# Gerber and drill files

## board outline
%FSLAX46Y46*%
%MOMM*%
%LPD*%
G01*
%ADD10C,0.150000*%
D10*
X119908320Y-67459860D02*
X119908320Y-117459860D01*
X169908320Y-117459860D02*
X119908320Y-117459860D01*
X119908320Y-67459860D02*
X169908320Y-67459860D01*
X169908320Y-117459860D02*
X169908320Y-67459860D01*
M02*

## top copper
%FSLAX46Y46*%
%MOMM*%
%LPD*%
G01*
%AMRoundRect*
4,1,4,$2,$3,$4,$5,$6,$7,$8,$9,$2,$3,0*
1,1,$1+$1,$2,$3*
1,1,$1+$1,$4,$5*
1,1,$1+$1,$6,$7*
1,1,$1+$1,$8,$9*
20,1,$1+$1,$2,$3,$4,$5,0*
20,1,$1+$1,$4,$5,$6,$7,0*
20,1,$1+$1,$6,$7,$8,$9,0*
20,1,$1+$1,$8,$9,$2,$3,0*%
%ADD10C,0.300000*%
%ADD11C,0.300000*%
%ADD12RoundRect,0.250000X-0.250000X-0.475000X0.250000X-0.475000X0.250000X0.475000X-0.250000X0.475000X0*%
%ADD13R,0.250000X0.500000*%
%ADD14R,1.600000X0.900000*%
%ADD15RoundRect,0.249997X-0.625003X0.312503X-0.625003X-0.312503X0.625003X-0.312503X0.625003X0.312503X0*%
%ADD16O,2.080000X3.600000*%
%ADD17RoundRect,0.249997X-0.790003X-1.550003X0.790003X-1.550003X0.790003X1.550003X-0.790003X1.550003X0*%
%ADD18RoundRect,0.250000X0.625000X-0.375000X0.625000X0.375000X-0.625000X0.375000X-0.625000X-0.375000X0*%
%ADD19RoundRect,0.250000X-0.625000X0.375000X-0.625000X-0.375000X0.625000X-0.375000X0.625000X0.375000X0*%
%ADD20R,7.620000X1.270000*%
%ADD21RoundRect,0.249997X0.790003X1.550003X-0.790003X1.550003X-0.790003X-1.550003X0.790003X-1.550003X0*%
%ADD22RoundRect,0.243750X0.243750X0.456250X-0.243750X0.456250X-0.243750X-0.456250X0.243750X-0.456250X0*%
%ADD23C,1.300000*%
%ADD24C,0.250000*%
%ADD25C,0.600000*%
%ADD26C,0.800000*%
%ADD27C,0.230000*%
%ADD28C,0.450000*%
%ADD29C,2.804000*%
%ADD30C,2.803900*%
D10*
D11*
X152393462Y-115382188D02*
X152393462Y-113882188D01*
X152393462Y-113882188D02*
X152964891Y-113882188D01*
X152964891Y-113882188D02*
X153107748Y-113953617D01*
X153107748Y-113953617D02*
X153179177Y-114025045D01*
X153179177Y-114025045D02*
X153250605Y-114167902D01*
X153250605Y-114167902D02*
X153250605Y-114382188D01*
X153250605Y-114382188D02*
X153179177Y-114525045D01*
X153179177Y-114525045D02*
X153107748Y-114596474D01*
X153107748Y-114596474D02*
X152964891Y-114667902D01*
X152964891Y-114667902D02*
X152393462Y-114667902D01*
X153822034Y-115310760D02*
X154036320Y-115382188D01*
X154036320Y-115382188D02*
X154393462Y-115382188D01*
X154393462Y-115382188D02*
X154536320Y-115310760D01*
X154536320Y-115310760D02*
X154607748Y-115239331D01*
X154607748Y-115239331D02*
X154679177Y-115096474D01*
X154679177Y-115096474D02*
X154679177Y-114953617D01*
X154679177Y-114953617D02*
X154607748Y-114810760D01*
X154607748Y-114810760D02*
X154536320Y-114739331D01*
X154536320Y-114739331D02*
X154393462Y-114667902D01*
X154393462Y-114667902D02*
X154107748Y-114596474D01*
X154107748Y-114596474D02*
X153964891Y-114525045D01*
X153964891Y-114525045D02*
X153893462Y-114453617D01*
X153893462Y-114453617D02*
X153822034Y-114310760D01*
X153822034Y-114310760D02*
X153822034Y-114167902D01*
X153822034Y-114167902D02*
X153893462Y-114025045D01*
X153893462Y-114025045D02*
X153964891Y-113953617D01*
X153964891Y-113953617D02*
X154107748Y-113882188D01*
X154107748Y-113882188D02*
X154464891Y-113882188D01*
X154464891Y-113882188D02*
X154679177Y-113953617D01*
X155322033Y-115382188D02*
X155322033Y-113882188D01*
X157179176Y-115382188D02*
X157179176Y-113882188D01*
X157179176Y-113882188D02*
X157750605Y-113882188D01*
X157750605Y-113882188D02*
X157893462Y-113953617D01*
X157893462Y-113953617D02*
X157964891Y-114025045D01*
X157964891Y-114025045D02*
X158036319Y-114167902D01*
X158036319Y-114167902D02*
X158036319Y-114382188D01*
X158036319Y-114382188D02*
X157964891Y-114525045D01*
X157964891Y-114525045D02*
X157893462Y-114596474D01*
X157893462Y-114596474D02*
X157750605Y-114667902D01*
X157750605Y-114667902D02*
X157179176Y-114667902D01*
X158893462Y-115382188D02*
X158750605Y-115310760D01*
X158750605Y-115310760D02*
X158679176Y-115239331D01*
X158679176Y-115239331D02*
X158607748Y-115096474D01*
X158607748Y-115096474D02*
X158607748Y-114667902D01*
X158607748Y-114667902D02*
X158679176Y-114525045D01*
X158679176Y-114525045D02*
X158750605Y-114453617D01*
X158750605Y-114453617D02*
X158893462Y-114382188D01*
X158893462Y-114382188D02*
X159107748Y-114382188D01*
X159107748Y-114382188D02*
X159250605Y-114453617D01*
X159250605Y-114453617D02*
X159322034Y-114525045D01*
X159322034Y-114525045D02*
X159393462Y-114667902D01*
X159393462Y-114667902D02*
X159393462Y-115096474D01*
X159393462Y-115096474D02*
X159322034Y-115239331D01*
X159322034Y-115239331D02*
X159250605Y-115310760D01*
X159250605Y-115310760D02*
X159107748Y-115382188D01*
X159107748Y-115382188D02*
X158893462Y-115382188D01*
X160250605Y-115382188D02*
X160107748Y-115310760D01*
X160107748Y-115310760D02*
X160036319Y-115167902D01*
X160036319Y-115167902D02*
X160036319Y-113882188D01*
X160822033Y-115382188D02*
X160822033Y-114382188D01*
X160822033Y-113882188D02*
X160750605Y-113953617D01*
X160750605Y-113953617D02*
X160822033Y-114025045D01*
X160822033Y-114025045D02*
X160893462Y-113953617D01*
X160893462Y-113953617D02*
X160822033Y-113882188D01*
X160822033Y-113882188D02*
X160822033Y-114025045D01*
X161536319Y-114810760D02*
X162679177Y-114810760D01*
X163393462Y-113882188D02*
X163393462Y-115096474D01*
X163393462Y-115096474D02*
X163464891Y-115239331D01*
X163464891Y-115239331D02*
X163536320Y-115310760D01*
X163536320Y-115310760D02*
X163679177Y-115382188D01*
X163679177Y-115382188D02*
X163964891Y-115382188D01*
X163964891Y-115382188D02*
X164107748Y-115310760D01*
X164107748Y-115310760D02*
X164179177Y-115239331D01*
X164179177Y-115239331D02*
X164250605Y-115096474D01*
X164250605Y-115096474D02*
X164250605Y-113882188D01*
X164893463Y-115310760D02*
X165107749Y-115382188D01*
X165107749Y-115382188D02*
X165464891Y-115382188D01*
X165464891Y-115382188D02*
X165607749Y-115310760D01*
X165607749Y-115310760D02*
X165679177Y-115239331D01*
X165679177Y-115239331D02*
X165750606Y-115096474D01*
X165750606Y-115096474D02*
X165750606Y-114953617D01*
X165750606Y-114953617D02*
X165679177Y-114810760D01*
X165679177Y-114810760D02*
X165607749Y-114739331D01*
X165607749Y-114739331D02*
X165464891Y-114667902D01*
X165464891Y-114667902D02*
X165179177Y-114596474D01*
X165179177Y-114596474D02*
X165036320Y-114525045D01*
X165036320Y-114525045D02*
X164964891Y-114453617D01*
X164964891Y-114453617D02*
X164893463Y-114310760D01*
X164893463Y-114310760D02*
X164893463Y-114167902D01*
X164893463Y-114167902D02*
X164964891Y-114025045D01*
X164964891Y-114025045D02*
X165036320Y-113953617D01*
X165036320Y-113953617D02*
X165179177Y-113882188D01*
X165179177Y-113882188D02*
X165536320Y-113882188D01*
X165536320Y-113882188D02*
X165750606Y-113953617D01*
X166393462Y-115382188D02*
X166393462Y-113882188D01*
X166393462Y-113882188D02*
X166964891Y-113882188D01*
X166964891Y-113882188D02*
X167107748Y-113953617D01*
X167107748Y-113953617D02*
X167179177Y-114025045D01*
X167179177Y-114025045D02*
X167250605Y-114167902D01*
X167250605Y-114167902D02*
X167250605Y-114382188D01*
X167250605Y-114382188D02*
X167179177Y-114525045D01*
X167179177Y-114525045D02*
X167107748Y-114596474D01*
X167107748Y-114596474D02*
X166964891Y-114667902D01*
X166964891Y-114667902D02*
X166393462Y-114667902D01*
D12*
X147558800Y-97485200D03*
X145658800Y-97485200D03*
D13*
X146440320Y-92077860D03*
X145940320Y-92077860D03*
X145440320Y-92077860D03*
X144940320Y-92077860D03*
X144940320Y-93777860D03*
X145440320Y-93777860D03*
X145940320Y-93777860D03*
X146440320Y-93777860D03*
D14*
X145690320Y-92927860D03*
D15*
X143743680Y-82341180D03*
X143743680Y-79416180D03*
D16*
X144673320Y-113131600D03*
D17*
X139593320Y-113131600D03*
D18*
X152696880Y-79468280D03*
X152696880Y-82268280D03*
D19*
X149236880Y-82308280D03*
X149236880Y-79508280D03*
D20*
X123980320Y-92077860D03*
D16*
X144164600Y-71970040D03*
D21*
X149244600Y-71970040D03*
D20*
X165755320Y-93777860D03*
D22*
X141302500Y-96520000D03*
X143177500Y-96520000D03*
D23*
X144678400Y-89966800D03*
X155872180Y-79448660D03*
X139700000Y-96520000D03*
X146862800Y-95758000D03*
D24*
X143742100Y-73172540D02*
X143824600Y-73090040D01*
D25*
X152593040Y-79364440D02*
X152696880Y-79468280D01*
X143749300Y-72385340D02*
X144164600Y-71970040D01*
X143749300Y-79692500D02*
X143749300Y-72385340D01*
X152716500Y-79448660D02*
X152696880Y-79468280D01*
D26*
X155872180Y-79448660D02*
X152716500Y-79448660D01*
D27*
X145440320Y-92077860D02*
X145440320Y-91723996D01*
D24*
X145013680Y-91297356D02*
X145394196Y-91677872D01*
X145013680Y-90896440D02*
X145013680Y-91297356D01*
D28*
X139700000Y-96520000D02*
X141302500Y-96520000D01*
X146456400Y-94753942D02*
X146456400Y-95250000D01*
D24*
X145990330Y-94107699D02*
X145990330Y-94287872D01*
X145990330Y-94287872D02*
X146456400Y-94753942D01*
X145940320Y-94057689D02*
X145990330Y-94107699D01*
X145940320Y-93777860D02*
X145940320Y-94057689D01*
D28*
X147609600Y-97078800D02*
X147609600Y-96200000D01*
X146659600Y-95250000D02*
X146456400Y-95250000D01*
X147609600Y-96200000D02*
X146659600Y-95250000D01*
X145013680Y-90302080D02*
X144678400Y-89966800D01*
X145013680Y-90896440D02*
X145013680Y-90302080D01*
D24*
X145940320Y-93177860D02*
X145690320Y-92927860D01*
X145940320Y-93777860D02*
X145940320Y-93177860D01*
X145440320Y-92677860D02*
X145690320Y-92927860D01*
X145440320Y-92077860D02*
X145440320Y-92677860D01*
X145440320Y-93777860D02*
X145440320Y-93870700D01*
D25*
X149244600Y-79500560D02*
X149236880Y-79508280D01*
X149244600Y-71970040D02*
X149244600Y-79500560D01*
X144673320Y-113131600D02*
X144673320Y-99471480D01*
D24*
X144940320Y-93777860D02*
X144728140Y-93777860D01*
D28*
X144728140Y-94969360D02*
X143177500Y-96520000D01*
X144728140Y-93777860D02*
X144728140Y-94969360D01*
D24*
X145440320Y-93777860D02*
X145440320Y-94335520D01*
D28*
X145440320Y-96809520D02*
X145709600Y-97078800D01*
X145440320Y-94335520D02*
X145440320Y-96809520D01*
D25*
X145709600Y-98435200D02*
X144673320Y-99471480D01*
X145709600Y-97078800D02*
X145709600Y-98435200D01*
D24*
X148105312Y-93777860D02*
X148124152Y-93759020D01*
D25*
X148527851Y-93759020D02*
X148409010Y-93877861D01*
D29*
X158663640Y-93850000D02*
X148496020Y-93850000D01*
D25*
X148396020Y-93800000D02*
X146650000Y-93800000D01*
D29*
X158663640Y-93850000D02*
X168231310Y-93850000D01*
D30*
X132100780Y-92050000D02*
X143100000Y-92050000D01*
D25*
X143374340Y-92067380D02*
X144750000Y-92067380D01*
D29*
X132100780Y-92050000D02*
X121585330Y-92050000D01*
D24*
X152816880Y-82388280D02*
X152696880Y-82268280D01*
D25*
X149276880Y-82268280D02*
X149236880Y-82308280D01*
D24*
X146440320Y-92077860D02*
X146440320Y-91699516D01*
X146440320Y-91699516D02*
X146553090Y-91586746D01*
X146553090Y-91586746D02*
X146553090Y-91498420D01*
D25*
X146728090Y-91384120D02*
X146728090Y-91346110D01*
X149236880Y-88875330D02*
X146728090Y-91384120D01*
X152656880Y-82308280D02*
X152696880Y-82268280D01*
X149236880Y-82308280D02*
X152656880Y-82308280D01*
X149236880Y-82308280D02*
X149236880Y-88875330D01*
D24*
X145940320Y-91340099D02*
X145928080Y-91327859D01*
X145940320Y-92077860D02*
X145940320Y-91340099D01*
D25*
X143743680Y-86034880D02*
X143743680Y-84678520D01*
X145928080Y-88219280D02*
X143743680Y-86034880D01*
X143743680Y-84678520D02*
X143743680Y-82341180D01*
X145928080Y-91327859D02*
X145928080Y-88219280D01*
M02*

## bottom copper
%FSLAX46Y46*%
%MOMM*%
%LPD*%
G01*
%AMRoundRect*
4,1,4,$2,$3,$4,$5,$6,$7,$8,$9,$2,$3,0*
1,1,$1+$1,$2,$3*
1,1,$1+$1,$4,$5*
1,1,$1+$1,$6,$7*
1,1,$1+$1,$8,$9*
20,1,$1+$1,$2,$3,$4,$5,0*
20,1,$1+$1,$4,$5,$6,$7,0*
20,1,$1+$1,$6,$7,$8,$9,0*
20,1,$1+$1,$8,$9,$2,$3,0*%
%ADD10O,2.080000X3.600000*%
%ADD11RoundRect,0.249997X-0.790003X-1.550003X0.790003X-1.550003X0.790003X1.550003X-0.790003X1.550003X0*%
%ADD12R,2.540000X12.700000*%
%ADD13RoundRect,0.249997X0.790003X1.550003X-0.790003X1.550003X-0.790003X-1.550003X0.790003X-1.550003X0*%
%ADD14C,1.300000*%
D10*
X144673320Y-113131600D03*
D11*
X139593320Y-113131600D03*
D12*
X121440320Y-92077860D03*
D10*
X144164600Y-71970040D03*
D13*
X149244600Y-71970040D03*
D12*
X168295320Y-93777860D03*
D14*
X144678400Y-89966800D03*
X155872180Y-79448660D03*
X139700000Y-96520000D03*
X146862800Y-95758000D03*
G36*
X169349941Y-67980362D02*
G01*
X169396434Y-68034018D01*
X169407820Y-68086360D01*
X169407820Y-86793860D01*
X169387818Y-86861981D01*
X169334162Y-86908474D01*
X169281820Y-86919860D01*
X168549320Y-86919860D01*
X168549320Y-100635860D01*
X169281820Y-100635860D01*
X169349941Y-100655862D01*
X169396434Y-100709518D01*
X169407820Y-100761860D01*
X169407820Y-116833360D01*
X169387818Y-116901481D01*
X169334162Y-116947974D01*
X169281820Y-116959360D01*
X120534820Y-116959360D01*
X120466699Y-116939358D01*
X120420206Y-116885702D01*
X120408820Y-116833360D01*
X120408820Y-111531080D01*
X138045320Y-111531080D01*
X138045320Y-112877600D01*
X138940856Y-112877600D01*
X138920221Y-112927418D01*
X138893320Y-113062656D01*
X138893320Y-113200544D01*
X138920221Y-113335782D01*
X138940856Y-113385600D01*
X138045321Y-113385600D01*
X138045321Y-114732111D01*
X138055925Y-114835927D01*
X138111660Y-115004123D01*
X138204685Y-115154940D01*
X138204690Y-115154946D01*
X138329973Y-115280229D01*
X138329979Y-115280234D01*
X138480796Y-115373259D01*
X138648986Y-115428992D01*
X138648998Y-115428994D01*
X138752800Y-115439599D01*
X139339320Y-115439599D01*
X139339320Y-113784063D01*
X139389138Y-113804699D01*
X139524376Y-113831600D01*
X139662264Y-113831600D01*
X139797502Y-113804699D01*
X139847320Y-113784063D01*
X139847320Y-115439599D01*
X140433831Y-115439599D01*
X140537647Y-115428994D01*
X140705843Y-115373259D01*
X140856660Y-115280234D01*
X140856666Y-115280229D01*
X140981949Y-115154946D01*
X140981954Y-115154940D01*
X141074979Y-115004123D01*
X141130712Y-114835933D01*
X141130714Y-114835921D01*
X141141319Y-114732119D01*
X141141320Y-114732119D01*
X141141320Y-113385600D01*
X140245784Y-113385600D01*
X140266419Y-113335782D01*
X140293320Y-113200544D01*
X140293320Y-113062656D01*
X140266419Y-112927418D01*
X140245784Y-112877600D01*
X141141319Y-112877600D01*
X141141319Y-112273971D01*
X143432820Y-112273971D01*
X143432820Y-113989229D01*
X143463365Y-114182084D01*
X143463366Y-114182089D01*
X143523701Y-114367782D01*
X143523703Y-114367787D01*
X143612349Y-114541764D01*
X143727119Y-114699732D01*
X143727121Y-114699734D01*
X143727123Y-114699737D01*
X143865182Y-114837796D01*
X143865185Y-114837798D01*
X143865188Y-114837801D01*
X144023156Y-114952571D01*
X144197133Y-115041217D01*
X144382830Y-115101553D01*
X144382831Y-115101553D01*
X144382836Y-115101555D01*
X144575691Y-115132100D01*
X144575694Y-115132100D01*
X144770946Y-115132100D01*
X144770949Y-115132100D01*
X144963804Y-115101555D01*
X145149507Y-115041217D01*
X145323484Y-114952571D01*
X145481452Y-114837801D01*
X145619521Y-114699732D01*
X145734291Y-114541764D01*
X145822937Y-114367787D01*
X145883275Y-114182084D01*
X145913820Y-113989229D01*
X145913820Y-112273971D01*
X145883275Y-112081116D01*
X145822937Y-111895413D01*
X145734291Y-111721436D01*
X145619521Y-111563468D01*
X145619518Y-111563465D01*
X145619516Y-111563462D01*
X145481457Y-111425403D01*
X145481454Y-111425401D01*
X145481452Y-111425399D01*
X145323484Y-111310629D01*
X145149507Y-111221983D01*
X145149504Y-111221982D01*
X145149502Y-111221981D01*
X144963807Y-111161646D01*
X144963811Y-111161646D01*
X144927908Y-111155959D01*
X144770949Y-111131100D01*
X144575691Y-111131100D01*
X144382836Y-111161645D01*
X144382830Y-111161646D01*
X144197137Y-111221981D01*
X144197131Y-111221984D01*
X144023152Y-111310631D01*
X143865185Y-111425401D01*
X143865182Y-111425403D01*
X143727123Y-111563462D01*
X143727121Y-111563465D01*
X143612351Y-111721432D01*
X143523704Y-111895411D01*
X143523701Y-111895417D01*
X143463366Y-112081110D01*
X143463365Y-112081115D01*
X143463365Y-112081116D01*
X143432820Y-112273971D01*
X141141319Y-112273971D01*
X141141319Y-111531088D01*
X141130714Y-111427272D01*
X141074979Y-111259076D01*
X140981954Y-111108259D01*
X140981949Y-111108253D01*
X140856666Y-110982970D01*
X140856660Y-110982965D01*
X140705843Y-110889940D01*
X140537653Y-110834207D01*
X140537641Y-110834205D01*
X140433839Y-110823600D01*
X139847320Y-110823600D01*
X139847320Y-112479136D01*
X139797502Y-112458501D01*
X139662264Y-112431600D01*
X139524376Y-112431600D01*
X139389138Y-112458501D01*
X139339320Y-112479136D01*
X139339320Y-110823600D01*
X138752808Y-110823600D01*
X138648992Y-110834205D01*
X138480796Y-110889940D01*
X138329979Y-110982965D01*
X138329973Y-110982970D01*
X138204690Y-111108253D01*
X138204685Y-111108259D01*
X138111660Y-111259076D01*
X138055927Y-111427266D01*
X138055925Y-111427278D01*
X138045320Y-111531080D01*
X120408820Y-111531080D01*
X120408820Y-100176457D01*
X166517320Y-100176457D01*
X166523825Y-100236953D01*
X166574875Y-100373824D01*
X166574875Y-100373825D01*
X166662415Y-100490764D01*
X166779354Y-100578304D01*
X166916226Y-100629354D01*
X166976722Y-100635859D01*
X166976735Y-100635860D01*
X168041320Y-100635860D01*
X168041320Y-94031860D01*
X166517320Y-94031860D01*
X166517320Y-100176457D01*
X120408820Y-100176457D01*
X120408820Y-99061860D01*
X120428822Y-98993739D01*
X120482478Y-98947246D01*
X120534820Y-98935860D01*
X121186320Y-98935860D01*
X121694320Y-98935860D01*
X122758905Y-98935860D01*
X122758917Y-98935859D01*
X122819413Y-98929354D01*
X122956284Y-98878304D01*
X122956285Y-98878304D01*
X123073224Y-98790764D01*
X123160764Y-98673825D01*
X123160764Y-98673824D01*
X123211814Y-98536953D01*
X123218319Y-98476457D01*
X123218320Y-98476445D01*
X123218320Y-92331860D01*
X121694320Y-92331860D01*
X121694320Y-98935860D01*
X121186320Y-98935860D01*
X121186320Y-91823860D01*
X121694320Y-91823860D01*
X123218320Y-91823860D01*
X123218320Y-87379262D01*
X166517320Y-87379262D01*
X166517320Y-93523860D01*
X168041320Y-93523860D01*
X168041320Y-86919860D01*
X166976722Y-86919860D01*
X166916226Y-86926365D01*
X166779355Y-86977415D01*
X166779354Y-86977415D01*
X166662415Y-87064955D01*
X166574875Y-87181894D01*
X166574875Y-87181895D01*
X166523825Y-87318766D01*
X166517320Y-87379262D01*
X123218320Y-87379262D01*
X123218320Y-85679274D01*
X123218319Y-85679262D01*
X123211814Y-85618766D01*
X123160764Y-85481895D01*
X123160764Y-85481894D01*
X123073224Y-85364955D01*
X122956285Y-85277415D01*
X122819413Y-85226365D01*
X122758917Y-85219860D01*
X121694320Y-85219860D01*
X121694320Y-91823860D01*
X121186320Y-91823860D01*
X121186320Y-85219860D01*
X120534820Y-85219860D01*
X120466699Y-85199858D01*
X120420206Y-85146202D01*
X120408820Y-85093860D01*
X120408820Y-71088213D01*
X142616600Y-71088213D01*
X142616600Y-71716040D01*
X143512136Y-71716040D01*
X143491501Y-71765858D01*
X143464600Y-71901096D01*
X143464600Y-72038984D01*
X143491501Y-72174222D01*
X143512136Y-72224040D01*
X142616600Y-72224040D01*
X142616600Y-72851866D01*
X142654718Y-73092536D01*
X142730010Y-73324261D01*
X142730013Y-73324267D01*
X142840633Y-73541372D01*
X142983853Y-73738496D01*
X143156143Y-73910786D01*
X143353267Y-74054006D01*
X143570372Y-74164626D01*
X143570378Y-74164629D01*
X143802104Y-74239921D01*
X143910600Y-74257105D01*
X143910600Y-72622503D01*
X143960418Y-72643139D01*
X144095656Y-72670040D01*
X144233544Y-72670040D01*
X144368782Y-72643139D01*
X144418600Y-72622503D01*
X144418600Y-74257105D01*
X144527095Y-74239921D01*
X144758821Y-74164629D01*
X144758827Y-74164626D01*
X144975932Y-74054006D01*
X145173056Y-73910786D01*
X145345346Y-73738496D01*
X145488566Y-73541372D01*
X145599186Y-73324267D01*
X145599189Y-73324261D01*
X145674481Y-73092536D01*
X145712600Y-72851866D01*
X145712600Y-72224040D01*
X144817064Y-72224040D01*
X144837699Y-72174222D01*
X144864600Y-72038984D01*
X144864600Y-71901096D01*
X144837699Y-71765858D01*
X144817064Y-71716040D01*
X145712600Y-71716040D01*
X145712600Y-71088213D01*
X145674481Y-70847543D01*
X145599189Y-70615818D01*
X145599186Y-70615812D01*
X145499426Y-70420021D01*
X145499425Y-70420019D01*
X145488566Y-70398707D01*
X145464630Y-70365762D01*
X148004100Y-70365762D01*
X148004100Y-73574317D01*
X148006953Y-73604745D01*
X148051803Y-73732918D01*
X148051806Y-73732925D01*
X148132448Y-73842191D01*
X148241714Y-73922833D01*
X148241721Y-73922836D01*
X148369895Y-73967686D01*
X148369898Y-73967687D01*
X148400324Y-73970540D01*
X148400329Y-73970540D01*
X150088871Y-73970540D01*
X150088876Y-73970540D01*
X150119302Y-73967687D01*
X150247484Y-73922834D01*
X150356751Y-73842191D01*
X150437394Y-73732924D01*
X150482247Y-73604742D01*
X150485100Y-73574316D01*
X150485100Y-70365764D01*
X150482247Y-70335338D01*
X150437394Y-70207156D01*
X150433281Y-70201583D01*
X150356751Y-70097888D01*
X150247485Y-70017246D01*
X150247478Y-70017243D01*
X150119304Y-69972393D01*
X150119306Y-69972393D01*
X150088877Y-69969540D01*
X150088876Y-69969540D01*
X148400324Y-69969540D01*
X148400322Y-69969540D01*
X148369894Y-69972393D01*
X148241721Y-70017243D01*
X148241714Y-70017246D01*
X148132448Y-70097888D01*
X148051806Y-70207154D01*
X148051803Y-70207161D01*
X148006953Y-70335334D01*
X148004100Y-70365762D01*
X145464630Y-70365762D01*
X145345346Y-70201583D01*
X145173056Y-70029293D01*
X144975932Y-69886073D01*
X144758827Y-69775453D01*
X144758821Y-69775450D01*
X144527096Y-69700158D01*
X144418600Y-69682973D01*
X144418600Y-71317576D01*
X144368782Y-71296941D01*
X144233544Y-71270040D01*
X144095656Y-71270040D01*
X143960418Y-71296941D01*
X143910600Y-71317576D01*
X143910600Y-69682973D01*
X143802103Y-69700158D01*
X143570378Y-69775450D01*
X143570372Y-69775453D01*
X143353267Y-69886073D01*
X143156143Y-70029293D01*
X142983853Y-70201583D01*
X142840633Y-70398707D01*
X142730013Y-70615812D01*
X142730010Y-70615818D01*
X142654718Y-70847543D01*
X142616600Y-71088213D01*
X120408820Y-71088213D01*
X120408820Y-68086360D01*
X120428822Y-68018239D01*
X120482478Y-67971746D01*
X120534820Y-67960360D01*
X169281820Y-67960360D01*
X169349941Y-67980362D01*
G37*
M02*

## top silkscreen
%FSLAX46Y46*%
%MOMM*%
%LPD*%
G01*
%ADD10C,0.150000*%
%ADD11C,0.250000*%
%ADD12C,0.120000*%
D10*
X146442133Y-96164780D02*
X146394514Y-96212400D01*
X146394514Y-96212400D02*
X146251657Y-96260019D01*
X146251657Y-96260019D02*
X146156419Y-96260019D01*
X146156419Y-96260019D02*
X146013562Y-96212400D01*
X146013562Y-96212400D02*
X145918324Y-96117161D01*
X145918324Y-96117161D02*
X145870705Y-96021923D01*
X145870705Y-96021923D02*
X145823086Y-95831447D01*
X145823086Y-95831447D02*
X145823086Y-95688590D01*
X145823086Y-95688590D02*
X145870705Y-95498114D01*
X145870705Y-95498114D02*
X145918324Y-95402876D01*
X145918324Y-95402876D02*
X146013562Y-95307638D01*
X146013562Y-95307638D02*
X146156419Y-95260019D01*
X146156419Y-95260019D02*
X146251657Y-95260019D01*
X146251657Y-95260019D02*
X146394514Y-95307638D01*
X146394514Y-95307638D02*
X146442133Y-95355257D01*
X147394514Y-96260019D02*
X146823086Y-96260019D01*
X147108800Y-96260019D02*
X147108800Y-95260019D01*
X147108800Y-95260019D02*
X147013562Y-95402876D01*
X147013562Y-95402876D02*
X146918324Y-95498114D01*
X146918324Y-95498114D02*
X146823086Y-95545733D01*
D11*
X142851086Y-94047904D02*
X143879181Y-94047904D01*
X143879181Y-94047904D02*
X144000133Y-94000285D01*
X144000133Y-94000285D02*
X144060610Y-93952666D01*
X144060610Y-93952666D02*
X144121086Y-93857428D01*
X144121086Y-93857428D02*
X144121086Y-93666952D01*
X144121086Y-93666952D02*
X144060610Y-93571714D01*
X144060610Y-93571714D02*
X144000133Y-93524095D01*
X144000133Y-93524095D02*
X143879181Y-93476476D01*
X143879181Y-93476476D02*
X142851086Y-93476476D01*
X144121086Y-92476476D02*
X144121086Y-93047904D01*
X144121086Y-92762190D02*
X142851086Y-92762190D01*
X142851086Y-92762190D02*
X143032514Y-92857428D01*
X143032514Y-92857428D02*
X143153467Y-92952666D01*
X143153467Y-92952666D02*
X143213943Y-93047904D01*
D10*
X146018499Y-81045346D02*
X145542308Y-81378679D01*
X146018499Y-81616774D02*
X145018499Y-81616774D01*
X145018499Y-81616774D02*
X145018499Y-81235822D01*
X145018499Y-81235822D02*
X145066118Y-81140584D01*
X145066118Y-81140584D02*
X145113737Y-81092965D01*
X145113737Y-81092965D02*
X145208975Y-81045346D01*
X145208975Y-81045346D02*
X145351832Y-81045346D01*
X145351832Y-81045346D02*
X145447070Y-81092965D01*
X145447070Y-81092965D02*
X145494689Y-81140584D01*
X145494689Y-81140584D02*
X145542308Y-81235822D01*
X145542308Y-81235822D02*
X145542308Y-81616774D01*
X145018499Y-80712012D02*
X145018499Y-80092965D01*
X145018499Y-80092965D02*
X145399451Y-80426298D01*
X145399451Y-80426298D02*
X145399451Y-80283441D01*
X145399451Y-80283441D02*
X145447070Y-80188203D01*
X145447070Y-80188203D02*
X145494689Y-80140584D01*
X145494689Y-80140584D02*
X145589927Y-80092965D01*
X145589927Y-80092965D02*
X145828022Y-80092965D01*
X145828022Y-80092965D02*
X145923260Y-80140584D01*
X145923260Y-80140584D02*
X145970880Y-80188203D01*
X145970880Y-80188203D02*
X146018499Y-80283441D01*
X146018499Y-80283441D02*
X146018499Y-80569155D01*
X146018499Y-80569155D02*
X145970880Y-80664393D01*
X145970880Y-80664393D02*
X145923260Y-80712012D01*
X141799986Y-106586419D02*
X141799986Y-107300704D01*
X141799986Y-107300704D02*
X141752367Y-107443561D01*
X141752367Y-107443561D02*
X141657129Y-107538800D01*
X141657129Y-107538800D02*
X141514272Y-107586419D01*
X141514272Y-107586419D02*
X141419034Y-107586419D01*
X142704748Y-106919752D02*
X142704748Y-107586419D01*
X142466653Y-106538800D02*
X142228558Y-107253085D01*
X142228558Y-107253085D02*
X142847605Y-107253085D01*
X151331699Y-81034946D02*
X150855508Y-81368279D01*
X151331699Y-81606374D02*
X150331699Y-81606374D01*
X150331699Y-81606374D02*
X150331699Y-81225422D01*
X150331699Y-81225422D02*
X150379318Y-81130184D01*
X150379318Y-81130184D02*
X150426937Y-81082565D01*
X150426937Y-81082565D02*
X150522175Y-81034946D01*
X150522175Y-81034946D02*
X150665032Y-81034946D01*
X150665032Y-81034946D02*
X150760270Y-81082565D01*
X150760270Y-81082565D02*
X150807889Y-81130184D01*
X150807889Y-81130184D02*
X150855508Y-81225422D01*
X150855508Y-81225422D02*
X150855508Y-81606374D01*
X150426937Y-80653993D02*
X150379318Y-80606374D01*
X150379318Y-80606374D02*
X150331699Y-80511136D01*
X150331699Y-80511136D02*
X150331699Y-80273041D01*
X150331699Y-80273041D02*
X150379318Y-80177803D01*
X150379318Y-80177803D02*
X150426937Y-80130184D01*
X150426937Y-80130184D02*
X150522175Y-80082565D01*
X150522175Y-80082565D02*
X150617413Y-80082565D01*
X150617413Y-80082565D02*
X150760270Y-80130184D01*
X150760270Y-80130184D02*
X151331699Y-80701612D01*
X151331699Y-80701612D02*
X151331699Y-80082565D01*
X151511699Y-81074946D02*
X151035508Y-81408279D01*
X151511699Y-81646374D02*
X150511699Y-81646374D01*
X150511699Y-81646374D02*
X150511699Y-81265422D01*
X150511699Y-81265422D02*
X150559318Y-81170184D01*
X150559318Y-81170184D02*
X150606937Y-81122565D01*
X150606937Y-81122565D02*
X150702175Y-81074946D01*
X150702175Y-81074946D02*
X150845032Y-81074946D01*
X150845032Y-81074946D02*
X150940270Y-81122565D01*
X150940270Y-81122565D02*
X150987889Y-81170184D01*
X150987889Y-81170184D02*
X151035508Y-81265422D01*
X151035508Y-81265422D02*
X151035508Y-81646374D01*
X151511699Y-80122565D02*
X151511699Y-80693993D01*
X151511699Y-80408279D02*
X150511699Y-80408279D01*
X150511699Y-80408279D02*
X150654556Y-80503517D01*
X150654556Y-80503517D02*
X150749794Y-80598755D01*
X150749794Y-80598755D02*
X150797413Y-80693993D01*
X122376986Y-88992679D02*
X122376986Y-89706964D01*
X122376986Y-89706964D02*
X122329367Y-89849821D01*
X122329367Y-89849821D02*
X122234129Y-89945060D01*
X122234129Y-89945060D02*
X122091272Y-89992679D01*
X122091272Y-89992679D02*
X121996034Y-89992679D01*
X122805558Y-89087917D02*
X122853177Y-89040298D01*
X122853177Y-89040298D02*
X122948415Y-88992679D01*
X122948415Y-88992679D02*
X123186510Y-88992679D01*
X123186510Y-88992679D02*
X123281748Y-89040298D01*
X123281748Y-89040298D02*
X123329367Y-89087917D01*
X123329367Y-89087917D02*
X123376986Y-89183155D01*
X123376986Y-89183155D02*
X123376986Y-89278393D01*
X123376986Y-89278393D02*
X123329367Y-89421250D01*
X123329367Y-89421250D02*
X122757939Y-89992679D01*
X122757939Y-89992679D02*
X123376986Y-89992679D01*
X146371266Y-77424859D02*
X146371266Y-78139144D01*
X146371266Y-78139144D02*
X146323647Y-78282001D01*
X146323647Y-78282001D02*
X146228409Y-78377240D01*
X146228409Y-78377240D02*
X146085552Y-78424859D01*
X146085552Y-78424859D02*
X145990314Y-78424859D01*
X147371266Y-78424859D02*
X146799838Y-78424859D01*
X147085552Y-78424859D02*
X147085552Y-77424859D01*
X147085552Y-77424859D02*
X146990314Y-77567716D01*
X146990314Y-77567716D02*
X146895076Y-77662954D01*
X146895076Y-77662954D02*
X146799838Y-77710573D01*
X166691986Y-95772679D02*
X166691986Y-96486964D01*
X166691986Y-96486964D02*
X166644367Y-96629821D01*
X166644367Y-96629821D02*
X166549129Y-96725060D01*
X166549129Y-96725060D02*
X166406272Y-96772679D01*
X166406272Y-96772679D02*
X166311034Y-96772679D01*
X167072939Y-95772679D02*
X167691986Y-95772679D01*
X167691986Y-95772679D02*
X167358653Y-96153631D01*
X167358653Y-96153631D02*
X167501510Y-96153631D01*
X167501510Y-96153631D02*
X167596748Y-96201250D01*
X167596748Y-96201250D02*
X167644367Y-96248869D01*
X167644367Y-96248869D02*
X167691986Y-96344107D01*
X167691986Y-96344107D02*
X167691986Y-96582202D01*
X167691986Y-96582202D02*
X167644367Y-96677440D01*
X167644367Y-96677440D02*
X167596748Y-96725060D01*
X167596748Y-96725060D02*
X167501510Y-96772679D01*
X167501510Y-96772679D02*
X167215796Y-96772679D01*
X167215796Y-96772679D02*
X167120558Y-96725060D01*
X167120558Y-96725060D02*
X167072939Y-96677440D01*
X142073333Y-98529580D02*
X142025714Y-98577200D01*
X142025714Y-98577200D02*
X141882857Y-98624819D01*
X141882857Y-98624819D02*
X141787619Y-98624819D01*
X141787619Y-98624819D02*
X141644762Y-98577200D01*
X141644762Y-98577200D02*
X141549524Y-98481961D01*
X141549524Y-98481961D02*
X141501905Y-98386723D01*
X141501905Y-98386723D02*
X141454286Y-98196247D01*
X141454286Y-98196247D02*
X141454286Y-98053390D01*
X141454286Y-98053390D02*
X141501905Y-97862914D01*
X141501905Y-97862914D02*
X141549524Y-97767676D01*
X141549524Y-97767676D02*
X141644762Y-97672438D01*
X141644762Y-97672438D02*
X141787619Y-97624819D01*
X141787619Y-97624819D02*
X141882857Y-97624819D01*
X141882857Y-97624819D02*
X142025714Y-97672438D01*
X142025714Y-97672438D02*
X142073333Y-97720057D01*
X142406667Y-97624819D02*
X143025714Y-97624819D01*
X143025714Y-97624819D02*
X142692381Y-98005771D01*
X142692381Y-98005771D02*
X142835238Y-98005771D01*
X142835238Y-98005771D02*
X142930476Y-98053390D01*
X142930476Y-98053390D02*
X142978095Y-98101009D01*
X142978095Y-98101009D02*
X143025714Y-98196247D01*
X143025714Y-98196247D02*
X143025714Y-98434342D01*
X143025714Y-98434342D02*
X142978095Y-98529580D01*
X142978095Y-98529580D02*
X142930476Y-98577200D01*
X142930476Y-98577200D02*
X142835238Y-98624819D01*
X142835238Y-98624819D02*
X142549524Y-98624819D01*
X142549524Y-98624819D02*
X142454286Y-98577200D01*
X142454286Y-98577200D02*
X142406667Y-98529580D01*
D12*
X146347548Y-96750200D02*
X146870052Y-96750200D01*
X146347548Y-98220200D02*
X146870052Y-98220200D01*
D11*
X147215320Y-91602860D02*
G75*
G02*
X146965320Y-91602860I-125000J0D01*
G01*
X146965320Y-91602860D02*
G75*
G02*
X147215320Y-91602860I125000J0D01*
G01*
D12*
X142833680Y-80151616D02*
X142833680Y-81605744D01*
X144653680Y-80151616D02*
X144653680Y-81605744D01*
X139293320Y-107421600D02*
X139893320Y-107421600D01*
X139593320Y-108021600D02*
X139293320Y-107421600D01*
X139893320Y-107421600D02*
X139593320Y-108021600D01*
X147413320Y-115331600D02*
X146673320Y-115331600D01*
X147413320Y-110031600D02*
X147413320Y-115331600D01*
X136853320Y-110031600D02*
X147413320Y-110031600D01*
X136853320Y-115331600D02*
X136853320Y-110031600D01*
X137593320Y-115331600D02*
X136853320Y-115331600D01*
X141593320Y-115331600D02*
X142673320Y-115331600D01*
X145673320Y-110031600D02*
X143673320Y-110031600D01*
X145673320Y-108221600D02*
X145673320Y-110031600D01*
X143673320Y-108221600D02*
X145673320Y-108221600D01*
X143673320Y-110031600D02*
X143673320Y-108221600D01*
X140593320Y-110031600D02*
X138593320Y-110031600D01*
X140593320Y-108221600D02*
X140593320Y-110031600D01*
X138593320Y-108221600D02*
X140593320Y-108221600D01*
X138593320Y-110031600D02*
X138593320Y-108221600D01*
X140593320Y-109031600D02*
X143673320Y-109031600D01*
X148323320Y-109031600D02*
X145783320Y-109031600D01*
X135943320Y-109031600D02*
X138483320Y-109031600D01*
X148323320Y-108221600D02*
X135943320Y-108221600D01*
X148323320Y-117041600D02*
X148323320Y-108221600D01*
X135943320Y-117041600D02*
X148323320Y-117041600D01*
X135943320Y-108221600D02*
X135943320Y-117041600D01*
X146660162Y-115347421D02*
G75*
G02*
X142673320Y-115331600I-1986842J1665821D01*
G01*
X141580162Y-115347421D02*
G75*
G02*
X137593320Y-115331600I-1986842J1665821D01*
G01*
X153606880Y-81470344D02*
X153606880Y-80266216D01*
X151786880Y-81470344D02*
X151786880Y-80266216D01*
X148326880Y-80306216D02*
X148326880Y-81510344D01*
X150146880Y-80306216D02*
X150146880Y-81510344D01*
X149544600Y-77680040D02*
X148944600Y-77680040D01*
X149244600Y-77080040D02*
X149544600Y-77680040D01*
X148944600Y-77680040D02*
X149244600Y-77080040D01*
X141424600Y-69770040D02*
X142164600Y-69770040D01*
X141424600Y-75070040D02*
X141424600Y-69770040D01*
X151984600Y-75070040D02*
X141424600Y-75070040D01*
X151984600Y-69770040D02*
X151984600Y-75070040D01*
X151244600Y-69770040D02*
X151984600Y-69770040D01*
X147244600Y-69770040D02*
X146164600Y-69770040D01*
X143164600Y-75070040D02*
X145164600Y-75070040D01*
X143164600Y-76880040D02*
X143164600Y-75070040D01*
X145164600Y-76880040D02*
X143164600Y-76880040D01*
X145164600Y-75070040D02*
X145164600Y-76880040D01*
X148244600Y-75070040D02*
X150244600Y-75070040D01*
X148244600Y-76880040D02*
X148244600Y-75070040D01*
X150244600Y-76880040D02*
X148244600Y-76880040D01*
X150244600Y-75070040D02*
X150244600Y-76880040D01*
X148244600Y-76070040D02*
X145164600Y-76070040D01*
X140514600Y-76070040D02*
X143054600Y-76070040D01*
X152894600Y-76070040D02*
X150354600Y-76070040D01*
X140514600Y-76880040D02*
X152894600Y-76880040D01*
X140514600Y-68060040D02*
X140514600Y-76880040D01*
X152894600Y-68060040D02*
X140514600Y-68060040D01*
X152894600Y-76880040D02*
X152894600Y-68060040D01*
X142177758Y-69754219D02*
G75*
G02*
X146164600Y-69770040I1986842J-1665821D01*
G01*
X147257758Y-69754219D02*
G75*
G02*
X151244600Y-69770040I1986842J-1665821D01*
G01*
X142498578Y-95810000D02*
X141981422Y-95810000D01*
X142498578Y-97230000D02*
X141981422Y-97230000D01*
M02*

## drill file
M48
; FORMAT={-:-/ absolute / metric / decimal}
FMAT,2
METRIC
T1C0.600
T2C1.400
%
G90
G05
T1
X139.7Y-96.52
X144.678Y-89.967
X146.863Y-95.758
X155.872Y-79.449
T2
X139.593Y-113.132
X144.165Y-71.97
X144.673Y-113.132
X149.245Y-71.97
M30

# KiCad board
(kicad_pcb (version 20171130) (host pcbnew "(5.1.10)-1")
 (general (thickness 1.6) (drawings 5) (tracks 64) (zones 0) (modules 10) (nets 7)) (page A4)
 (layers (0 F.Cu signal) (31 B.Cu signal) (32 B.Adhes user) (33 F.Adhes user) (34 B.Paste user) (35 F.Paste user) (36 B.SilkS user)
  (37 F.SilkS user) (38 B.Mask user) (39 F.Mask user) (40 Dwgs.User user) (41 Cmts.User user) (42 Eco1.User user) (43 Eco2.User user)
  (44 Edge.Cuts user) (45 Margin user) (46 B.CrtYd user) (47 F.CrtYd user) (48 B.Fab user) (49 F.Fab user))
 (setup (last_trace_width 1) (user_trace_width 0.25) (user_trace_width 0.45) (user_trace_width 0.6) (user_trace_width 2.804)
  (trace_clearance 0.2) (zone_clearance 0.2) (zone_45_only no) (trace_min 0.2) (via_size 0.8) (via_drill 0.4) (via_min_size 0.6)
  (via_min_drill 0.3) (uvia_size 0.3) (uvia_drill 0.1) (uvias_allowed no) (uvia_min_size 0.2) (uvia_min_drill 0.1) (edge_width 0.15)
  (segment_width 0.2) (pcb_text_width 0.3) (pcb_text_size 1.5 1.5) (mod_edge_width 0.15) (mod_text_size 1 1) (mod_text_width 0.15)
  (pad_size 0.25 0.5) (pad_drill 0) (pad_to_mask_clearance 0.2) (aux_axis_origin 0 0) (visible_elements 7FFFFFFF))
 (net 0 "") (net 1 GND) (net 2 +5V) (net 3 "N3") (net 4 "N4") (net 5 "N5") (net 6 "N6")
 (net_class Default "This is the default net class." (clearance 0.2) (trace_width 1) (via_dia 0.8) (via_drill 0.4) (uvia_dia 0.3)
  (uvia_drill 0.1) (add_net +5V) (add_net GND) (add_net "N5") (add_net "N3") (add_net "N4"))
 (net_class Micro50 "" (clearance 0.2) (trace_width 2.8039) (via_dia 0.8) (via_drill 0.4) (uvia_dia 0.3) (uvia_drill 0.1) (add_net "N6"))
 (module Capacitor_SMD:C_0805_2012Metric (layer F.Cu) (at 146.6088 97.4852)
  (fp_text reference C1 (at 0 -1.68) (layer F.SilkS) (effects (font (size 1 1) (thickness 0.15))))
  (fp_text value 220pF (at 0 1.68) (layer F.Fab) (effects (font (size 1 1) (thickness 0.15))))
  (fp_line (start -0.261252 -0.735) (end 0.261252 -0.735) (layer F.SilkS) (width 0.12))
  (fp_line (start -0.261252 0.735) (end 0.261252 0.735) (layer F.SilkS) (width 0.12))
  (pad 2 smd roundrect (at 0.95 0) (size 1 1.45) (layers F.Cu F.Paste F.Mask) (roundrect_rratio 0.25) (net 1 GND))
  (pad 1 smd roundrect (at -0.95 0) (size 1 1.45) (layers F.Cu F.Paste F.Mask) (roundrect_rratio 0.25) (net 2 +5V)))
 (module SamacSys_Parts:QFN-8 (layer F.Cu) (at 145.69032 92.92786 270)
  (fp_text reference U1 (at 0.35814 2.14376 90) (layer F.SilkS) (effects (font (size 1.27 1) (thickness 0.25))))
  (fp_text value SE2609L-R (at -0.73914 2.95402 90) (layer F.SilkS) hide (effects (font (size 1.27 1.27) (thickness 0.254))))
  (fp_circle (center -1.325 -1.4) (end -1.325 -1.275) (layer F.SilkS) (width 0.25))
  (pad 1 smd rect (at -0.85 -0.75) (size 0.25 0.5) (layers F.Cu F.Paste F.Mask) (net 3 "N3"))
  (pad 2 smd rect (at -0.85 -0.25) (size 0.25 0.5) (layers F.Cu F.Paste F.Mask) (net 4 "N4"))
  (pad 3 smd rect (at -0.85 0.25) (size 0.25 0.5) (layers F.Cu F.Paste F.Mask) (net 1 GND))
  (pad 4 smd rect (at -0.85 0.75) (size 0.25 0.5) (layers F.Cu F.Paste F.Mask) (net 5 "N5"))
  (pad 5 smd rect (at 0.85 0.75) (size 0.25 0.5) (layers F.Cu F.Paste F.Mask) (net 2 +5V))
  (pad 6 smd rect (at 0.85 0.25) (size 0.25 0.5) (layers F.Cu F.Paste F.Mask) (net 2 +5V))
  (pad 7 smd rect (at 0.85 -0.25) (size 0.25 0.5) (layers F.Cu F.Paste F.Mask) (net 1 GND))
  (pad 8 smd rect (at 0.85 -0.75) (size 0.25 0.5) (layers F.Cu F.Paste F.Mask) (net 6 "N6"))
  (pad 9 smd rect (at 0 0 270) (size 0.9 1.6) (layers F.Cu F.Paste F.Mask) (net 1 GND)))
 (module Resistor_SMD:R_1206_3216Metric (layer F.Cu) (at 143.74368 80.87868 270)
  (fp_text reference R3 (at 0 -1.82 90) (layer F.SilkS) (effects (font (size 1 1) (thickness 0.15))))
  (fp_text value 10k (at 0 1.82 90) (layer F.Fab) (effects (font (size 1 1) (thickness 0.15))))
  (fp_line (start -0.727064 0.91) (end 0.727064 0.91) (layer F.SilkS) (width 0.12))
  (fp_line (start -0.727064 -0.91) (end 0.727064 -0.91) (layer F.SilkS) (width 0.12))
  (pad 2 smd roundrect (at 1.4625 0 270) (size 1.125 1.75) (layers F.Cu F.Paste F.Mask) (roundrect_rratio 0.2222195555555556) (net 4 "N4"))
  (pad 1 smd roundrect (at -1.4625 0 270) (size 1.125 1.75) (layers F.Cu F.Paste F.Mask) (roundrect_rratio 0.2222195555555556) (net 1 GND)))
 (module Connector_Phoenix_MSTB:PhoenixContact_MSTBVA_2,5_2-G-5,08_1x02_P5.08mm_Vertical (layer F.Cu) (at 139.59332 113.1316)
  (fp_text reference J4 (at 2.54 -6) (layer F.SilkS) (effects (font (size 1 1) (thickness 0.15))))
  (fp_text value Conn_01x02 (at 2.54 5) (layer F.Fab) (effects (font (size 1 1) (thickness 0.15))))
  (fp_line (start -0.3 -5.71) (end 0.3 -5.71) (layer F.SilkS) (width 0.12))
  (fp_line (start 0 -5.11) (end -0.3 -5.71) (layer F.SilkS) (width 0.12))
  (fp_line (start 0.3 -5.71) (end 0 -5.11) (layer F.SilkS) (width 0.12))
  (fp_line (start 7.82 2.2) (end 7.08 2.2) (layer F.SilkS) (width 0.12))
  (fp_line (start 7.82 -3.1) (end 7.82 2.2) (layer F.SilkS) (width 0.12))
  (fp_line (start -2.74 -3.1) (end 7.82 -3.1) (layer F.SilkS) (width 0.12))
  (fp_line (start -2.74 2.2) (end -2.74 -3.1) (layer F.SilkS) (width 0.12))
  (fp_line (start -2 2.2) (end -2.74 2.2) (layer F.SilkS) (width 0.12))
  (fp_line (start 2 2.2) (end 3.08 2.2) (layer F.SilkS) (width 0.12))
  (fp_line (start 6.08 -3.1) (end 4.08 -3.1) (layer F.SilkS) (width 0.12))
  (fp_line (start 6.08 -4.91) (end 6.08 -3.1) (layer F.SilkS) (width 0.12))
  (fp_line (start 4.08 -4.91) (end 6.08 -4.91) (layer F.SilkS) (width 0.12))
  (fp_line (start 4.08 -3.1) (end 4.08 -4.91) (layer F.SilkS) (width 0.12))
  (fp_line (start 1 -3.1) (end -1 -3.1) (layer F.SilkS) (width 0.12))
  (fp_line (start 1 -4.91) (end 1 -3.1) (layer F.SilkS) (width 0.12))
  (fp_line (start -1 -4.91) (end 1 -4.91) (layer F.SilkS) (width 0.12))
  (fp_line (start -1 -3.1) (end -1 -4.91) (layer F.SilkS) (width 0.12))
  (fp_line (start 1 -4.1) (end 4.08 -4.1) (layer F.SilkS) (width 0.12))
  (fp_line (start 8.73 -4.1) (end 6.19 -4.1) (layer F.SilkS) (width 0.12))
  (fp_line (start -3.65 -4.1) (end -1.11 -4.1) (layer F.SilkS) (width 0.12))
  (fp_line (start 8.73 -4.91) (end -3.65 -4.91) (layer F.SilkS) (width 0.12))
  (fp_line (start 8.73 3.91) (end 8.73 -4.91) (layer F.SilkS) (width 0.12))
  (fp_line (start -3.65 3.91) (end 8.73 3.91) (layer F.SilkS) (width 0.12))
  (fp_line (start -3.65 -4.91) (end -3.65 3.91) (layer F.SilkS) (width 0.12))
  (fp_arc (start 5.08 0.55) (end 3.08 2.2) (angle -100.5) (layer F.SilkS) (width 0.12))
  (fp_arc (start 0 0.55) (end -2 2.2) (angle -100.5) (layer F.SilkS) (width 0.12))
  (pad 2 thru_hole oval (at 5.08 0) (size 2.08 3.6) (drill 1.4) (layers *.Cu *.Mask) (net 2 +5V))
  (pad 1 thru_hole roundrect (at 0 0) (size 2.08 3.6) (drill 1.4) (layers *.Cu *.Mask) (roundrect_rratio 0.1201908653846154) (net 1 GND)))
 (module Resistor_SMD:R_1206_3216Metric (layer F.Cu) (at 152.69688 80.86828 90)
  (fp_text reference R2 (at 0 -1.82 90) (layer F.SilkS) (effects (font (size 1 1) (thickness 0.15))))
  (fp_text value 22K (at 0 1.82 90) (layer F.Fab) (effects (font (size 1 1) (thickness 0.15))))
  (fp_line (start -0.602064 0.91) (end 0.602064 0.91) (layer F.SilkS) (width 0.12))
  (fp_line (start -0.602064 -0.91) (end 0.602064 -0.91) (layer F.SilkS) (width 0.12))
  (pad 2 smd roundrect (at 1.4 0 90) (size 1.25 1.75) (layers F.Cu F.Paste F.Mask) (roundrect_rratio 0.2) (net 1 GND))
  (pad 1 smd roundrect (at -1.4 0 90) (size 1.25 1.75) (layers F.Cu F.Paste F.Mask) (roundrect_rratio 0.2) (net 3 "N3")))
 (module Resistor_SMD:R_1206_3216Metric (layer F.Cu) (at 149.23688 80.90828 270)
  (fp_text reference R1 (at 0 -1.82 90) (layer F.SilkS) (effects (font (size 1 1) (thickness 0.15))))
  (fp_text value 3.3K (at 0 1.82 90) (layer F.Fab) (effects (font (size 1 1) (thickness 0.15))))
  (fp_line (start -0.602064 0.91) (end 0.602064 0.91) (layer F.SilkS) (width 0.12))
  (fp_line (start -0.602064 -0.91) (end 0.602064 -0.91) (layer F.SilkS) (width 0.12))
  (pad 2 smd roundrect (at 1.4 0 270) (size 1.25 1.75) (layers F.Cu F.Paste F.Mask) (roundrect_rratio 0.2) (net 3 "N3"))
  (pad 1 smd roundrect (at -1.4 0 270) (size 1.25 1.75) (layers F.Cu F.Paste F.Mask) (roundrect_rratio 0.2) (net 2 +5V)))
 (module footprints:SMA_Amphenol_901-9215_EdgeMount (layer F.Cu) (at 125.25032 92.07786 180)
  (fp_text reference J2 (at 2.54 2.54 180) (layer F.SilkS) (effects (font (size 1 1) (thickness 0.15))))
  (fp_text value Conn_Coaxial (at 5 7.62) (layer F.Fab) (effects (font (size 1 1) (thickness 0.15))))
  (pad 1 smd rect (at 1.27 0 270) (size 1.27 7.62) (layers F.Cu F.Paste F.Mask) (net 5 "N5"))
  (pad 2 smd rect (at 3.81 0) (size 2.54 12.7) (layers B.Cu B.Paste B.Mask) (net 1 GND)))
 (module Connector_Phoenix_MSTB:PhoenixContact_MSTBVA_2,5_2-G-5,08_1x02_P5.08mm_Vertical (layer F.Cu) (at 149.2446 71.97004 180)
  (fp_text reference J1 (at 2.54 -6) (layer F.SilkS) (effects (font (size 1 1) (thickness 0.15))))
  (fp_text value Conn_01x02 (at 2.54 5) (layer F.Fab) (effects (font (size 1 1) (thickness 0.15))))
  (fp_line (start -0.3 -5.71) (end 0.3 -5.71) (layer F.SilkS) (width 0.12))
  (fp_line (start 0 -5.11) (end -0.3 -5.71) (layer F.SilkS) (width 0.12))
  (fp_line (start 0.3 -5.71) (end 0 -5.11) (layer F.SilkS) (width 0.12))
  (fp_line (start 7.82 2.2) (end 7.08 2.2) (layer F.SilkS) (width 0.12))
  (fp_line (start 7.82 -3.1) (end 7.82 2.2) (layer F.SilkS) (width 0.12))
  (fp_line (start -2.74 -3.1) (end 7.82 -3.1) (layer F.SilkS) (width 0.12))
  (fp_line (start -2.74 2.2) (end -2.74 -3.1) (layer F.SilkS) (width 0.12))
  (fp_line (start -2 2.2) (end -2.74 2.2) (layer F.SilkS) (width 0.12))
  (fp_line (start 2 2.2) (end 3.08 2.2) (layer F.SilkS) (width 0.12))
  (fp_line (start 6.08 -3.1) (end 4.08 -3.1) (layer F.SilkS) (width 0.12))
  (fp_line (start 6.08 -4.91) (end 6.08 -3.1) (layer F.SilkS) (width 0.12))
  (fp_line (start 4.08 -4.91) (end 6.08 -4.91) (layer F.SilkS) (width 0.12))
  (fp_line (start 4.08 -3.1) (end 4.08 -4.91) (layer F.SilkS) (width 0.12))
  (fp_line (start 1 -3.1) (end -1 -3.1) (layer F.SilkS) (width 0.12))
  (fp_line (start 1 -4.91) (end 1 -3.1) (layer F.SilkS) (width 0.12))
  (fp_line (start -1 -4.91) (end 1 -4.91) (layer F.SilkS) (width 0.12))
  (fp_line (start -1 -3.1) (end -1 -4.91) (layer F.SilkS) (width 0.12))
  (fp_line (start 1 -4.1) (end 4.08 -4.1) (layer F.SilkS) (width 0.12))
  (fp_line (start 8.73 -4.1) (end 6.19 -4.1) (layer F.SilkS) (width 0.12))
  (fp_line (start -3.65 -4.1) (end -1.11 -4.1) (layer F.SilkS) (width 0.12))
  (fp_line (start 8.73 -4.91) (end -3.65 -4.91) (layer F.SilkS) (width 0.12))
  (fp_line (start 8.73 3.91) (end 8.73 -4.91) (layer F.SilkS) (width 0.12))
  (fp_line (start -3.65 3.91) (end 8.73 3.91) (layer F.SilkS) (width 0.12))
  (fp_line (start -3.65 -4.91) (end -3.65 3.91) (layer F.SilkS) (width 0.12))
  (fp_arc (start 5.08 0.55) (end 3.08 2.2) (angle -100.5) (layer F.SilkS) (width 0.12))
  (fp_arc (start 0 0.55) (end -2 2.2) (angle -100.5) (layer F.SilkS) (width 0.12))
  (pad 2 thru_hole oval (at 5.08 0 180) (size 2.08 3.6) (drill 1.4) (layers *.Cu *.Mask) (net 1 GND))
  (pad 1 thru_hole roundrect (at 0 0 180) (size 2.08 3.6) (drill 1.4) (layers *.Cu *.Mask) (roundrect_rratio 0.1201908653846154) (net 2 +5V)))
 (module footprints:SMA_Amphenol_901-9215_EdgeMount (layer F.Cu) (at 164.48532 93.77786)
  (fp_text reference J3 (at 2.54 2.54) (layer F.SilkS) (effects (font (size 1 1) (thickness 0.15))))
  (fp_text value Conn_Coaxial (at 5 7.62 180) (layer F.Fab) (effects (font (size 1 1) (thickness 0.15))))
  (pad 1 smd rect (at 1.27 0 90) (size 1.27 7.62) (layers F.Cu F.Paste F.Mask) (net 6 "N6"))
  (pad 2 smd rect (at 3.81 0 180) (size 2.54 12.7) (layers B.Cu B.Paste B.Mask) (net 1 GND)))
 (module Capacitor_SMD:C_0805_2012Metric (layer F.Cu) (at 142.24 96.52 180)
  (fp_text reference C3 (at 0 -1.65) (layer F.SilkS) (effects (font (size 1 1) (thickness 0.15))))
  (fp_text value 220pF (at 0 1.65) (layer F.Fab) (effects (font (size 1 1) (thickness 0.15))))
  (fp_line (start -0.258578 0.71) (end 0.258578 0.71) (layer F.SilkS) (width 0.12))
  (fp_line (start -0.258578 -0.71) (end 0.258578 -0.71) (layer F.SilkS) (width 0.12))
  (pad 2 smd roundrect (at 0.9375 0 180) (size 0.975 1.4) (layers F.Cu F.Paste F.Mask) (roundrect_rratio 0.25) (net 1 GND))
  (pad 1 smd roundrect (at -0.9375 0 180) (size 0.975 1.4) (layers F.Cu F.Paste F.Mask) (roundrect_rratio 0.25) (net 2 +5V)))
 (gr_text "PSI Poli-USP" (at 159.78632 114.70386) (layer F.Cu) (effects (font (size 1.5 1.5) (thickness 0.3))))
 (gr_line (start 119.90832 67.45986) (end 119.90832 117.45986) (layer Edge.Cuts) (width 0.15))
 (gr_line (start 169.90832 117.45986) (end 119.90832 117.45986) (layer Edge.Cuts) (width 0.15))
 (gr_line (start 119.90832 67.45986) (end 169.90832 67.45986) (layer Edge.Cuts) (width 0.15))
 (gr_line (start 169.90832 117.45986) (end 169.90832 67.45986) (layer Edge.Cuts) (width 0.15))
 (via (at 144.6784 89.9668) (size 1.3) (drill 0.6) (layers F.Cu B.Cu) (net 1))
 (via (at 155.87218 79.44866) (size 1.3) (drill 0.6) (layers F.Cu B.Cu) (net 1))
 (segment (start 143.7421 73.17254) (end 143.8246 73.09004) (width 0.25) (layer F.Cu) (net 1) (status 30))
 (segment (start 152.59304 79.36444) (end 152.69688 79.46828) (width 0.6) (layer F.Cu) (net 1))
 (segment (start 143.7493 72.38534) (end 144.1646 71.97004) (width 0.6) (layer F.Cu) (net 1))
 (segment (start 143.7493 79.6925) (end 143.7493 72.38534) (width 0.6) (layer F.Cu) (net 1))
 (segment (start 152.7165 79.44866) (end 152.69688 79.46828) (width 0.6) (layer F.Cu) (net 1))
 (segment (start 155.87218 79.44866) (end 152.7165 79.44866) (width 0.8) (layer F.Cu) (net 1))
 (segment (start 145.44032 92.07786) (end 145.44032 91.723996) (width 0.23) (layer F.Cu) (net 1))
 (segment (start 145.01368 91.297356) (end 145.394196 91.677872) (width 0.25) (layer F.Cu) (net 1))
 (segment (start 145.01368 90.89644) (end 145.01368 91.297356) (width 0.25) (layer F.Cu) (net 1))
 (via (at 139.7 96.52) (size 1.3) (drill 0.6) (layers F.Cu B.Cu) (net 1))
 (via (at 146.8628 95.758) (size 1.3) (drill 0.6) (layers F.Cu B.Cu) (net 1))
 (segment (start 139.7 96.52) (end 141.3025 96.52) (width 0.45) (layer F.Cu) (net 1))
 (segment (start 146.4564 94.753942) (end 146.4564 95.25) (width 0.45) (layer F.Cu) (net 1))
 (segment (start 145.99033 94.107699) (end 145.99033 94.287872) (width 0.25) (layer F.Cu) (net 1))
 (segment (start 145.99033 94.287872) (end 146.4564 94.753942) (width 0.25) (layer F.Cu) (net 1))
 (segment (start 145.94032 94.057689) (end 145.99033 94.107699) (width 0.25) (layer F.Cu) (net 1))
 (segment (start 145.94032 93.77786) (end 145.94032 94.057689) (width 0.25) (layer F.Cu) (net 1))
 (segment (start 147.6096 97.0788) (end 147.6096 96.2) (width 0.45) (layer F.Cu) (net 1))
 (segment (start 146.6596 95.25) (end 146.4564 95.25) (width 0.45) (layer F.Cu) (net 1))
 (segment (start 147.6096 96.2) (end 146.6596 95.25) (width 0.45) (layer F.Cu) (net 1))
 (segment (start 145.01368 90.30208) (end 144.6784 89.9668) (width 0.45) (layer F.Cu) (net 1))
 (segment (start 145.01368 90.89644) (end 145.01368 90.30208) (width 0.45) (layer F.Cu) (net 1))
 (segment (start 145.94032 93.17786) (end 145.69032 92.92786) (width 0.25) (layer F.Cu) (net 1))
 (segment (start 145.94032 93.77786) (end 145.94032 93.17786) (width 0.25) (layer F.Cu) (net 1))
 (segment (start 145.44032 92.67786) (end 145.69032 92.92786) (width 0.25) (layer F.Cu) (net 1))
 (segment (start 145.44032 92.07786) (end 145.44032 92.67786) (width 0.25) (layer F.Cu) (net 1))
 (segment (start 145.44032 93.77786) (end 145.44032 93.8707) (width 0.25) (layer F.Cu) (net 2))
 (segment (start 149.2446 79.50056) (end 149.23688 79.50828) (width 0.6) (layer F.Cu) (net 2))
 (segment (start 149.2446 71.97004) (end 149.2446 79.50056) (width 0.6) (layer F.Cu) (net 2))
 (segment (start 144.67332 113.1316) (end 144.67332 99.47148) (width 0.6) (layer F.Cu) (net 2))
 (segment (start 144.94032 93.77786) (end 144.72814 93.77786) (width 0.25) (layer F.Cu) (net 2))
 (segment (start 144.72814 94.96936) (end 143.1775 96.52) (width 0.45) (layer F.Cu) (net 2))
 (segment (start 144.72814 93.77786) (end 144.72814 94.96936) (width 0.45) (layer F.Cu) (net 2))
 (segment (start 145.44032 93.77786) (end 145.44032 94.33552) (width 0.25) (layer F.Cu) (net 2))
 (segment (start 145.44032 96.80952) (end 145.7096 97.0788) (width 0.45) (layer F.Cu) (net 2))
 (segment (start 145.44032 94.33552) (end 145.44032 96.80952) (width 0.45) (layer F.Cu) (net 2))
 (segment (start 145.7096 98.4352) (end 144.67332 99.47148) (width 0.6) (layer F.Cu) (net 2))
 (segment (start 145.7096 97.0788) (end 145.7096 98.4352) (width 0.6) (layer F.Cu) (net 2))
 (segment (start 148.105312 93.77786) (end 148.124152 93.75902) (width 0.25) (layer F.Cu) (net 6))
 (segment (start 148.527851 93.75902) (end 148.40901 93.877861) (width 0.6) (layer F.Cu) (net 6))
 (segment (start 158.66364 93.85) (end 148.49602 93.85) (width 2.804) (layer F.Cu) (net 6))
 (segment (start 148.39602 93.8) (end 146.65 93.8) (width 0.6) (layer F.Cu) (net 6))
 (segment (start 158.66364 93.85) (end 168.23131 93.85) (width 2.804) (layer F.Cu) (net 6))
 (segment (start 132.10078 92.05) (end 143.1 92.05) (width 2.8039) (layer F.Cu) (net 5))
 (segment (start 143.37434 92.06738) (end 144.75 92.06738) (width 0.6) (layer F.Cu) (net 5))
 (segment (start 132.10078 92.05) (end 121.58533 92.05) (width 2.804) (layer F.Cu) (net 5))
 (segment (start 152.81688 82.38828) (end 152.69688 82.26828) (width 0.25) (layer F.Cu) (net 3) (status 30))
 (segment (start 149.27688 82.26828) (end 149.23688 82.30828) (width 0.6) (layer F.Cu) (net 3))
 (segment (start 146.44032 92.07786) (end 146.44032 91.699516) (width 0.25) (layer F.Cu) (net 3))
 (segment (start 146.44032 91.699516) (end 146.55309 91.586746) (width 0.25) (layer F.Cu) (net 3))
 (segment (start 146.55309 91.586746) (end 146.55309 91.49842) (width 0.25) (layer F.Cu) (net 3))
 (segment (start 146.72809 91.38412) (end 146.72809 91.34611) (width 0.6) (layer F.Cu) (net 3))
 (segment (start 149.23688 88.87533) (end 146.72809 91.38412) (width 0.6) (layer F.Cu) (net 3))
 (segment (start 152.65688 82.30828) (end 152.69688 82.26828) (width 0.6) (layer F.Cu) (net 3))
 (segment (start 149.23688 82.30828) (end 152.65688 82.30828) (width 0.6) (layer F.Cu) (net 3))
 (segment (start 149.23688 82.30828) (end 149.23688 88.87533) (width 0.6) (layer F.Cu) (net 3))
 (segment (start 145.94032 91.340099) (end 145.92808 91.327859) (width 0.25) (layer F.Cu) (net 4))
 (segment (start 145.94032 92.07786) (end 145.94032 91.340099) (width 0.25) (layer F.Cu) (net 4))
 (segment (start 143.74368 86.03488) (end 143.74368 84.67852) (width 0.6) (layer F.Cu) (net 4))
 (segment (start 145.92808 88.21928) (end 143.74368 86.03488) (width 0.6) (layer F.Cu) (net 4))
 (segment (start 143.74368 84.67852) (end 143.74368 82.34118) (width 0.6) (layer F.Cu) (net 4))
 (segment (start 145.92808 91.327859) (end 145.92808 88.21928) (width 0.6) (layer F.Cu) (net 4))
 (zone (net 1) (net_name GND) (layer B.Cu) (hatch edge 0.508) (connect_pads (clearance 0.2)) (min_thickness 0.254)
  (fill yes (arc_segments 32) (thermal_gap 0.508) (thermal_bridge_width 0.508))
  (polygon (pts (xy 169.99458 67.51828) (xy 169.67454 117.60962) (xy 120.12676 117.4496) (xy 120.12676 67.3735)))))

